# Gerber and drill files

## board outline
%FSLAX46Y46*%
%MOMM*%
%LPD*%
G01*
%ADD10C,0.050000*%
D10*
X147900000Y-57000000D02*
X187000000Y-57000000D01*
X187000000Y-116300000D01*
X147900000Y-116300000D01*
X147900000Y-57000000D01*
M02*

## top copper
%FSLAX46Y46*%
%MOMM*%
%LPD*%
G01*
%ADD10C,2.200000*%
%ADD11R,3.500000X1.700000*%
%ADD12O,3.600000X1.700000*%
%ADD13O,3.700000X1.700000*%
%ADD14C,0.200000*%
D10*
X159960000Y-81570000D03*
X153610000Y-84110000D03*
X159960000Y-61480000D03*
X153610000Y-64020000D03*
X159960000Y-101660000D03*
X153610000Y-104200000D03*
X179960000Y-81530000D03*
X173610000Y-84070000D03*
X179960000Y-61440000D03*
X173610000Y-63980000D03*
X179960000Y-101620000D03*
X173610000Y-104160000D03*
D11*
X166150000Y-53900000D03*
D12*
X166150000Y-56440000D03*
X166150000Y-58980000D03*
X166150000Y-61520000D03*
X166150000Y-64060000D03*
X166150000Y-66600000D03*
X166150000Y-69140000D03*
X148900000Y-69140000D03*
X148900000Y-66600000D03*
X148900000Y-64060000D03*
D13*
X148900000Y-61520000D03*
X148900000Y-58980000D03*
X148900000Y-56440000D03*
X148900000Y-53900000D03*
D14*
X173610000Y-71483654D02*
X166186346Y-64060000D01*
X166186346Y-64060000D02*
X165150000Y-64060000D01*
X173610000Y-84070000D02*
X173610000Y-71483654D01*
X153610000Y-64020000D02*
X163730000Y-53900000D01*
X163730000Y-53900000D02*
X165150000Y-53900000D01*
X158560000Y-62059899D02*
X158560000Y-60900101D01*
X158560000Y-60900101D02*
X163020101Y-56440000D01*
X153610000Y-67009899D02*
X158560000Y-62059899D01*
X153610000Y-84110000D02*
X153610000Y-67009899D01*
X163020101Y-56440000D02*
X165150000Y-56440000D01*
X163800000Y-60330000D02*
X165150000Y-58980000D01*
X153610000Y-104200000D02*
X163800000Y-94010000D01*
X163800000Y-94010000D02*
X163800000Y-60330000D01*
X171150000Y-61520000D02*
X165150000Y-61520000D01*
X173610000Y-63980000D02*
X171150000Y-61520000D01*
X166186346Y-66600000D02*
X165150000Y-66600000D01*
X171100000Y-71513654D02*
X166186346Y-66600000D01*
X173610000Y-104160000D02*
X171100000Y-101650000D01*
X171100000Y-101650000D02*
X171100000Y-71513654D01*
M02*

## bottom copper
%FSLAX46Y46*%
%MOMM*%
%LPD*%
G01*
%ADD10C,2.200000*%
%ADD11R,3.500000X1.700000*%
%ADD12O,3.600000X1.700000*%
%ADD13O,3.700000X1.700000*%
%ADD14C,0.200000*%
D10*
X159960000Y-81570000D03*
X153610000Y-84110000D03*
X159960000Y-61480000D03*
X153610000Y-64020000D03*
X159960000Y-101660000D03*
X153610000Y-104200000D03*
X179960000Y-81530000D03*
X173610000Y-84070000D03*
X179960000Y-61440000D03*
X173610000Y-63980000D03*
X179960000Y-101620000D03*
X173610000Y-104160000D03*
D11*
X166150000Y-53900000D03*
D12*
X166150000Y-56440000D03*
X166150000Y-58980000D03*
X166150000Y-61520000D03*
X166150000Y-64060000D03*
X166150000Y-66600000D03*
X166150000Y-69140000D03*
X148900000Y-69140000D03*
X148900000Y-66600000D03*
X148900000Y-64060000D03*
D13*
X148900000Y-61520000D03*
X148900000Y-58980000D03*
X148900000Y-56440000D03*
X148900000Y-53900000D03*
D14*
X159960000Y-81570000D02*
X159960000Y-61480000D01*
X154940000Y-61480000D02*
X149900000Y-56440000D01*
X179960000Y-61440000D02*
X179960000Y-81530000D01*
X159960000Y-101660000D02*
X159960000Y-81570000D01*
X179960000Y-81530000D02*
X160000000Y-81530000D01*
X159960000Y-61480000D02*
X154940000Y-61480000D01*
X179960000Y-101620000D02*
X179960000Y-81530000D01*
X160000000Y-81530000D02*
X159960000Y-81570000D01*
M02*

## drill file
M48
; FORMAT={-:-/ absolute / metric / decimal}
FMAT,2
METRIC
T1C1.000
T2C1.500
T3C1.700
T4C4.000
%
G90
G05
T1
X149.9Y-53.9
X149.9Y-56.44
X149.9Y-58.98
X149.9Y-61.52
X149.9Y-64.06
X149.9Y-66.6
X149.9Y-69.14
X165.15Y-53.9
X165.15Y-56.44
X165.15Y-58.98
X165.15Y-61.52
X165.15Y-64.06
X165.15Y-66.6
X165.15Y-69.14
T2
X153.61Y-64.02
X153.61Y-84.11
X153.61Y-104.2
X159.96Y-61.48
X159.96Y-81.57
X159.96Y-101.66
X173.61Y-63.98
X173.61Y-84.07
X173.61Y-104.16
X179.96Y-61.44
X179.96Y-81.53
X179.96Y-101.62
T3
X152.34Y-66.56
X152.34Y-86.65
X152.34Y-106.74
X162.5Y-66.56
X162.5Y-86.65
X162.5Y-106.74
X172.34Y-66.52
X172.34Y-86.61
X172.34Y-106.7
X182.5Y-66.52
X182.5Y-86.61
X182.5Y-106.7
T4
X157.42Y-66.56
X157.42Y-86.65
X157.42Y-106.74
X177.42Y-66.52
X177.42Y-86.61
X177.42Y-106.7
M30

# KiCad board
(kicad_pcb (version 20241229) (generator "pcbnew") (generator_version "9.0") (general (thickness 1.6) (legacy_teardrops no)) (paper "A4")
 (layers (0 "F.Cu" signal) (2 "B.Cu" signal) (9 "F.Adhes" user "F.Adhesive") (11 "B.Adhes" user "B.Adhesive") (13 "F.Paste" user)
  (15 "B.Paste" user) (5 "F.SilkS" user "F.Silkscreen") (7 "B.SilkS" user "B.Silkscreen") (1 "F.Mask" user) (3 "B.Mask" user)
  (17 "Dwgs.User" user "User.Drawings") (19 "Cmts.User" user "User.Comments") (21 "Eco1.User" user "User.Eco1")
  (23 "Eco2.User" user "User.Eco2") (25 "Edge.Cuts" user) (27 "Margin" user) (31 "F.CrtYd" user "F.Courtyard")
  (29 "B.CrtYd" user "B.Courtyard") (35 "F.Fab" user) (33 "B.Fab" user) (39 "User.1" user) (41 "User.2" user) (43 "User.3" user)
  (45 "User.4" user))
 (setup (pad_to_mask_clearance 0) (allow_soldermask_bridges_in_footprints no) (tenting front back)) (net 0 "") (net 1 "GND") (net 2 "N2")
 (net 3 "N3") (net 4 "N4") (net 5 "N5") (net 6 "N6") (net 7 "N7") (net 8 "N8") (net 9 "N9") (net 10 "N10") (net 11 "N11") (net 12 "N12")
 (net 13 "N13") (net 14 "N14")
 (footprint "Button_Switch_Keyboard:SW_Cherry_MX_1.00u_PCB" (layer "F.Cu") (at 159.96 81.57)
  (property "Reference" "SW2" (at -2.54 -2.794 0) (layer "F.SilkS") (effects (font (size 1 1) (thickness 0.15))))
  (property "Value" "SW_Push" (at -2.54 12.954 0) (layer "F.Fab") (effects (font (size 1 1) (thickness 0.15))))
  (pad "" np_thru_hole circle (at -7.62 5.08) (size 1.7 1.7) (drill 1.7) (layers "*.Cu" "*.Mask"))
  (pad "" np_thru_hole circle (at -2.54 5.08) (size 4 4) (drill 4) (layers "*.Cu" "*.Mask"))
  (pad "" np_thru_hole circle (at 2.54 5.08) (size 1.7 1.7) (drill 1.7) (layers "*.Cu" "*.Mask"))
  (pad "1" thru_hole circle (at 0 0) (size 2.2 2.2) (drill 1.5) (layers "*.Cu" "*.Mask") (remove_unused_layers no) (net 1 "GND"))
  (pad "2" thru_hole circle (at -6.35 2.54) (size 2.2 2.2) (drill 1.5) (layers "*.Cu" "*.Mask") (remove_unused_layers no) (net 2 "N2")))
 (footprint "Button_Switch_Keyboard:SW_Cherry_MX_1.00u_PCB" (layer "F.Cu") (at 159.96 61.48)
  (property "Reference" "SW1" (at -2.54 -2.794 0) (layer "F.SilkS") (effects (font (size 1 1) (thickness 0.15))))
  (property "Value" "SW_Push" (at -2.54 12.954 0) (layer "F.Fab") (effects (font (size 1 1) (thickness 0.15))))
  (pad "" np_thru_hole circle (at -7.62 5.08) (size 1.7 1.7) (drill 1.7) (layers "*.Cu" "*.Mask"))
  (pad "" np_thru_hole circle (at -2.54 5.08) (size 4 4) (drill 4) (layers "*.Cu" "*.Mask"))
  (pad "" np_thru_hole circle (at 2.54 5.08) (size 1.7 1.7) (drill 1.7) (layers "*.Cu" "*.Mask"))
  (pad "1" thru_hole circle (at 0 0) (size 2.2 2.2) (drill 1.5) (layers "*.Cu" "*.Mask") (remove_unused_layers no) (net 1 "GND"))
  (pad "2" thru_hole circle (at -6.35 2.54) (size 2.2 2.2) (drill 1.5) (layers "*.Cu" "*.Mask") (remove_unused_layers no) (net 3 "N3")))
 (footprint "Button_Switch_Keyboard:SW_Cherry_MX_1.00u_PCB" (layer "F.Cu") (at 159.96 101.66)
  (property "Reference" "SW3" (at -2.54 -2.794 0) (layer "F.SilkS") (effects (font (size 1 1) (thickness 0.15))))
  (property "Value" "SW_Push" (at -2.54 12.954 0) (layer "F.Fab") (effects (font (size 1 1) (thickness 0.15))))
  (pad "" np_thru_hole circle (at -7.62 5.08) (size 1.7 1.7) (drill 1.7) (layers "*.Cu" "*.Mask"))
  (pad "" np_thru_hole circle (at -2.54 5.08) (size 4 4) (drill 4) (layers "*.Cu" "*.Mask"))
  (pad "" np_thru_hole circle (at 2.54 5.08) (size 1.7 1.7) (drill 1.7) (layers "*.Cu" "*.Mask"))
  (pad "1" thru_hole circle (at 0 0) (size 2.2 2.2) (drill 1.5) (layers "*.Cu" "*.Mask") (remove_unused_layers no) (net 1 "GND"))
  (pad "2" thru_hole circle (at -6.35 2.54) (size 2.2 2.2) (drill 1.5) (layers "*.Cu" "*.Mask") (remove_unused_layers no) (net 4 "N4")))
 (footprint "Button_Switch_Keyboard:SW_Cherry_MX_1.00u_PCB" (layer "F.Cu") (at 179.96 81.53)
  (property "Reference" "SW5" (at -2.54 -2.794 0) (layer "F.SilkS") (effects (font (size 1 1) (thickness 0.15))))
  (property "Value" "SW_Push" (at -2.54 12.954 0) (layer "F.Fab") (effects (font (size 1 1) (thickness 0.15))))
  (pad "" np_thru_hole circle (at -7.62 5.08) (size 1.7 1.7) (drill 1.7) (layers "*.Cu" "*.Mask"))
  (pad "" np_thru_hole circle (at -2.54 5.08) (size 4 4) (drill 4) (layers "*.Cu" "*.Mask"))
  (pad "" np_thru_hole circle (at 2.54 5.08) (size 1.7 1.7) (drill 1.7) (layers "*.Cu" "*.Mask"))
  (pad "1" thru_hole circle (at 0 0) (size 2.2 2.2) (drill 1.5) (layers "*.Cu" "*.Mask") (remove_unused_layers no) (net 1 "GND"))
  (pad "2" thru_hole circle (at -6.35 2.54) (size 2.2 2.2) (drill 1.5) (layers "*.Cu" "*.Mask") (remove_unused_layers no) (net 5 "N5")))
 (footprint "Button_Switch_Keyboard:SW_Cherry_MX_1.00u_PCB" (layer "F.Cu") (at 179.96 61.44)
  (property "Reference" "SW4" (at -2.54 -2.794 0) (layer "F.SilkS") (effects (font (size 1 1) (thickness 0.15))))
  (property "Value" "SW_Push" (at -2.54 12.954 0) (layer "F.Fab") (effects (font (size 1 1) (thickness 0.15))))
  (pad "" np_thru_hole circle (at -7.62 5.08) (size 1.7 1.7) (drill 1.7) (layers "*.Cu" "*.Mask"))
  (pad "" np_thru_hole circle (at -2.54 5.08) (size 4 4) (drill 4) (layers "*.Cu" "*.Mask"))
  (pad "" np_thru_hole circle (at 2.54 5.08) (size 1.7 1.7) (drill 1.7) (layers "*.Cu" "*.Mask"))
  (pad "1" thru_hole circle (at 0 0) (size 2.2 2.2) (drill 1.5) (layers "*.Cu" "*.Mask") (remove_unused_layers no) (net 1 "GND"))
  (pad "2" thru_hole circle (at -6.35 2.54) (size 2.2 2.2) (drill 1.5) (layers "*.Cu" "*.Mask") (remove_unused_layers no) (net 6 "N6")))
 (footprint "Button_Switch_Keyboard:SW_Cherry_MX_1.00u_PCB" (layer "F.Cu") (at 179.96 101.62)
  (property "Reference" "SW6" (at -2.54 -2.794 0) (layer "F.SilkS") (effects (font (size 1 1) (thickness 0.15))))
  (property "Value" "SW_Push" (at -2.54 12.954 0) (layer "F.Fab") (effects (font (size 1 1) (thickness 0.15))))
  (pad "" np_thru_hole circle (at -7.62 5.08) (size 1.7 1.7) (drill 1.7) (layers "*.Cu" "*.Mask"))
  (pad "" np_thru_hole circle (at -2.54 5.08) (size 4 4) (drill 4) (layers "*.Cu" "*.Mask"))
  (pad "" np_thru_hole circle (at 2.54 5.08) (size 1.7 1.7) (drill 1.7) (layers "*.Cu" "*.Mask"))
  (pad "1" thru_hole circle (at 0 0) (size 2.2 2.2) (drill 1.5) (layers "*.Cu" "*.Mask") (remove_unused_layers no) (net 1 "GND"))
  (pad "2" thru_hole circle (at -6.35 2.54) (size 2.2 2.2) (drill 1.5) (layers "*.Cu" "*.Mask") (remove_unused_layers no) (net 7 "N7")))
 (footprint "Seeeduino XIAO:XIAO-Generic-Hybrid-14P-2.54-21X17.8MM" (layer "B.Cu") (at 157.525 61.52 180)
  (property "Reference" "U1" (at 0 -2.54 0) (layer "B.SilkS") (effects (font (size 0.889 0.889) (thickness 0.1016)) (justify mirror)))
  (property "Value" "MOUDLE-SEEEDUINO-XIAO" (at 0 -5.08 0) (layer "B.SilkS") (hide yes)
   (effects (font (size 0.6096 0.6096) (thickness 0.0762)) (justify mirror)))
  (pad "1" thru_hole rect (at -7.625 7.62 180) (size 3.5 1.7) (drill 1 (offset -1 0)) (layers "*.Cu" "*.Mask") (remove_unused_layers no)
   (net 3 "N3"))
  (pad "2" thru_hole oval (at -7.625 5.08 180) (size 3.6 1.7) (drill 1 (offset -1 0)) (layers "*.Cu" "*.Mask") (remove_unused_layers no)
   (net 2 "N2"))
  (pad "3" thru_hole oval (at -7.625 2.54 180) (size 3.6 1.7) (drill 1 (offset -1 0)) (layers "*.Cu" "*.Mask") (remove_unused_layers no)
   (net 4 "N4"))
  (pad "4" thru_hole oval (at -7.625 0 180) (size 3.6 1.7) (drill 1 (offset -1 0)) (layers "*.Cu" "*.Mask") (remove_unused_layers no)
   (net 6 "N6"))
  (pad "5" thru_hole oval (at -7.625 -2.54 180) (size 3.6 1.7) (drill 1 (offset -1 0)) (layers "*.Cu" "*.Mask") (remove_unused_layers no)
   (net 5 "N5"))
  (pad "6" thru_hole oval (at -7.625 -5.08) (size 3.6 1.7) (drill 1 (offset 1 0)) (layers "*.Cu" "*.Mask") (remove_unused_layers no)
   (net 7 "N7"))
  (pad "7" thru_hole oval (at -7.625 -7.62 180) (size 3.6 1.7) (drill 1 (offset -1 0)) (layers "*.Cu" "*.Mask") (remove_unused_layers no)
   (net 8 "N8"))
  (pad "8" thru_hole oval (at 7.625 -7.62 180) (size 3.6 1.7) (drill 1 (offset 1 0)) (layers "*.Cu" "*.Mask") (remove_unused_layers no)
   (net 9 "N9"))
  (pad "9" thru_hole oval (at 7.625 -5.08 180) (size 3.6 1.7) (drill 1 (offset 1 0)) (layers "*.Cu" "*.Mask") (remove_unused_layers no)
   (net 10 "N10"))
  (pad "10" thru_hole oval (at 7.625 -2.54 180) (size 3.6 1.7) (drill 1 (offset 1 0)) (layers "*.Cu" "*.Mask") (remove_unused_layers no)
   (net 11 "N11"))
  (pad "11" thru_hole oval (at 7.625 0 180) (size 3.7 1.7) (drill 1 (offset 1 0)) (layers "*.Cu" "*.Mask") (remove_unused_layers no)
   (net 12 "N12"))
  (pad "12" thru_hole oval (at 7.625 2.54 180) (size 3.7 1.7) (drill 1 (offset 1 0)) (layers "*.Cu" "*.Mask") (remove_unused_layers no)
   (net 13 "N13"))
  (pad "13" thru_hole oval (at 7.625 5.08 180) (size 3.7 1.7) (drill 1 (offset 1 0)) (layers "*.Cu" "*.Mask") (remove_unused_layers no)
   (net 1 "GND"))
  (pad "14" thru_hole oval (at 7.625 7.62 180) (size 3.7 1.7) (drill 1 (offset 1 0)) (layers "*.Cu" "*.Mask") (remove_unused_layers no)
   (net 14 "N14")))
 (gr_rect (start 147.9 57) (end 187 116.3) (stroke (width 0.05) (type default)) (fill no) (layer "Edge.Cuts"))
 (segment (start 159.96 81.57) (end 159.96 61.48) (width 0.2) (layer "B.Cu") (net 1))
 (segment (start 154.94 61.48) (end 149.9 56.44) (width 0.2) (layer "B.Cu") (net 1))
 (segment (start 179.96 61.44) (end 179.96 81.53) (width 0.2) (layer "B.Cu") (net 1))
 (segment (start 159.96 101.66) (end 159.96 81.57) (width 0.2) (layer "B.Cu") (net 1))
 (segment (start 179.96 81.53) (end 160 81.53) (width 0.2) (layer "B.Cu") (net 1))
 (segment (start 159.96 61.48) (end 154.94 61.48) (width 0.2) (layer "B.Cu") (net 1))
 (segment (start 179.96 101.62) (end 179.96 81.53) (width 0.2) (layer "B.Cu") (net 1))
 (segment (start 160 81.53) (end 159.96 81.57) (width 0.2) (layer "B.Cu") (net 1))
 (segment (start 173.61 71.483654) (end 166.186346 64.06) (width 0.2) (layer "F.Cu") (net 5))
 (segment (start 166.186346 64.06) (end 165.15 64.06) (width 0.2) (layer "F.Cu") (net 5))
 (segment (start 173.61 84.07) (end 173.61 71.483654) (width 0.2) (layer "F.Cu") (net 5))
 (segment (start 153.61 64.02) (end 163.73 53.9) (width 0.2) (layer "F.Cu") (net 3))
 (segment (start 163.73 53.9) (end 165.15 53.9) (width 0.2) (layer "F.Cu") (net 3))
 (segment (start 158.56 62.059899) (end 158.56 60.900101) (width 0.2) (layer "F.Cu") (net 2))
 (segment (start 158.56 60.900101) (end 163.020101 56.44) (width 0.2) (layer "F.Cu") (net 2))
 (segment (start 153.61 67.009899) (end 158.56 62.059899) (width 0.2) (layer "F.Cu") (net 2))
 (segment (start 153.61 84.11) (end 153.61 67.009899) (width 0.2) (layer "F.Cu") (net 2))
 (segment (start 163.020101 56.44) (end 165.15 56.44) (width 0.2) (layer "F.Cu") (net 2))
 (segment (start 163.8 60.33) (end 165.15 58.98) (width 0.2) (layer "F.Cu") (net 4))
 (segment (start 153.61 104.2) (end 163.8 94.01) (width 0.2) (layer "F.Cu") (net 4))
 (segment (start 163.8 94.01) (end 163.8 60.33) (width 0.2) (layer "F.Cu") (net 4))
 (segment (start 171.15 61.52) (end 165.15 61.52) (width 0.2) (layer "F.Cu") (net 6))
 (segment (start 173.61 63.98) (end 171.15 61.52) (width 0.2) (layer "F.Cu") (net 6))
 (segment (start 166.186346 66.6) (end 165.15 66.6) (width 0.2) (layer "F.Cu") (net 7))
 (segment (start 171.1 71.513654) (end 166.186346 66.6) (width 0.2) (layer "F.Cu") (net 7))
 (segment (start 173.61 104.16) (end 171.1 101.65) (width 0.2) (layer "F.Cu") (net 7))
 (segment (start 171.1 101.65) (end 171.1 71.513654) (width 0.2) (layer "F.Cu") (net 7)))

